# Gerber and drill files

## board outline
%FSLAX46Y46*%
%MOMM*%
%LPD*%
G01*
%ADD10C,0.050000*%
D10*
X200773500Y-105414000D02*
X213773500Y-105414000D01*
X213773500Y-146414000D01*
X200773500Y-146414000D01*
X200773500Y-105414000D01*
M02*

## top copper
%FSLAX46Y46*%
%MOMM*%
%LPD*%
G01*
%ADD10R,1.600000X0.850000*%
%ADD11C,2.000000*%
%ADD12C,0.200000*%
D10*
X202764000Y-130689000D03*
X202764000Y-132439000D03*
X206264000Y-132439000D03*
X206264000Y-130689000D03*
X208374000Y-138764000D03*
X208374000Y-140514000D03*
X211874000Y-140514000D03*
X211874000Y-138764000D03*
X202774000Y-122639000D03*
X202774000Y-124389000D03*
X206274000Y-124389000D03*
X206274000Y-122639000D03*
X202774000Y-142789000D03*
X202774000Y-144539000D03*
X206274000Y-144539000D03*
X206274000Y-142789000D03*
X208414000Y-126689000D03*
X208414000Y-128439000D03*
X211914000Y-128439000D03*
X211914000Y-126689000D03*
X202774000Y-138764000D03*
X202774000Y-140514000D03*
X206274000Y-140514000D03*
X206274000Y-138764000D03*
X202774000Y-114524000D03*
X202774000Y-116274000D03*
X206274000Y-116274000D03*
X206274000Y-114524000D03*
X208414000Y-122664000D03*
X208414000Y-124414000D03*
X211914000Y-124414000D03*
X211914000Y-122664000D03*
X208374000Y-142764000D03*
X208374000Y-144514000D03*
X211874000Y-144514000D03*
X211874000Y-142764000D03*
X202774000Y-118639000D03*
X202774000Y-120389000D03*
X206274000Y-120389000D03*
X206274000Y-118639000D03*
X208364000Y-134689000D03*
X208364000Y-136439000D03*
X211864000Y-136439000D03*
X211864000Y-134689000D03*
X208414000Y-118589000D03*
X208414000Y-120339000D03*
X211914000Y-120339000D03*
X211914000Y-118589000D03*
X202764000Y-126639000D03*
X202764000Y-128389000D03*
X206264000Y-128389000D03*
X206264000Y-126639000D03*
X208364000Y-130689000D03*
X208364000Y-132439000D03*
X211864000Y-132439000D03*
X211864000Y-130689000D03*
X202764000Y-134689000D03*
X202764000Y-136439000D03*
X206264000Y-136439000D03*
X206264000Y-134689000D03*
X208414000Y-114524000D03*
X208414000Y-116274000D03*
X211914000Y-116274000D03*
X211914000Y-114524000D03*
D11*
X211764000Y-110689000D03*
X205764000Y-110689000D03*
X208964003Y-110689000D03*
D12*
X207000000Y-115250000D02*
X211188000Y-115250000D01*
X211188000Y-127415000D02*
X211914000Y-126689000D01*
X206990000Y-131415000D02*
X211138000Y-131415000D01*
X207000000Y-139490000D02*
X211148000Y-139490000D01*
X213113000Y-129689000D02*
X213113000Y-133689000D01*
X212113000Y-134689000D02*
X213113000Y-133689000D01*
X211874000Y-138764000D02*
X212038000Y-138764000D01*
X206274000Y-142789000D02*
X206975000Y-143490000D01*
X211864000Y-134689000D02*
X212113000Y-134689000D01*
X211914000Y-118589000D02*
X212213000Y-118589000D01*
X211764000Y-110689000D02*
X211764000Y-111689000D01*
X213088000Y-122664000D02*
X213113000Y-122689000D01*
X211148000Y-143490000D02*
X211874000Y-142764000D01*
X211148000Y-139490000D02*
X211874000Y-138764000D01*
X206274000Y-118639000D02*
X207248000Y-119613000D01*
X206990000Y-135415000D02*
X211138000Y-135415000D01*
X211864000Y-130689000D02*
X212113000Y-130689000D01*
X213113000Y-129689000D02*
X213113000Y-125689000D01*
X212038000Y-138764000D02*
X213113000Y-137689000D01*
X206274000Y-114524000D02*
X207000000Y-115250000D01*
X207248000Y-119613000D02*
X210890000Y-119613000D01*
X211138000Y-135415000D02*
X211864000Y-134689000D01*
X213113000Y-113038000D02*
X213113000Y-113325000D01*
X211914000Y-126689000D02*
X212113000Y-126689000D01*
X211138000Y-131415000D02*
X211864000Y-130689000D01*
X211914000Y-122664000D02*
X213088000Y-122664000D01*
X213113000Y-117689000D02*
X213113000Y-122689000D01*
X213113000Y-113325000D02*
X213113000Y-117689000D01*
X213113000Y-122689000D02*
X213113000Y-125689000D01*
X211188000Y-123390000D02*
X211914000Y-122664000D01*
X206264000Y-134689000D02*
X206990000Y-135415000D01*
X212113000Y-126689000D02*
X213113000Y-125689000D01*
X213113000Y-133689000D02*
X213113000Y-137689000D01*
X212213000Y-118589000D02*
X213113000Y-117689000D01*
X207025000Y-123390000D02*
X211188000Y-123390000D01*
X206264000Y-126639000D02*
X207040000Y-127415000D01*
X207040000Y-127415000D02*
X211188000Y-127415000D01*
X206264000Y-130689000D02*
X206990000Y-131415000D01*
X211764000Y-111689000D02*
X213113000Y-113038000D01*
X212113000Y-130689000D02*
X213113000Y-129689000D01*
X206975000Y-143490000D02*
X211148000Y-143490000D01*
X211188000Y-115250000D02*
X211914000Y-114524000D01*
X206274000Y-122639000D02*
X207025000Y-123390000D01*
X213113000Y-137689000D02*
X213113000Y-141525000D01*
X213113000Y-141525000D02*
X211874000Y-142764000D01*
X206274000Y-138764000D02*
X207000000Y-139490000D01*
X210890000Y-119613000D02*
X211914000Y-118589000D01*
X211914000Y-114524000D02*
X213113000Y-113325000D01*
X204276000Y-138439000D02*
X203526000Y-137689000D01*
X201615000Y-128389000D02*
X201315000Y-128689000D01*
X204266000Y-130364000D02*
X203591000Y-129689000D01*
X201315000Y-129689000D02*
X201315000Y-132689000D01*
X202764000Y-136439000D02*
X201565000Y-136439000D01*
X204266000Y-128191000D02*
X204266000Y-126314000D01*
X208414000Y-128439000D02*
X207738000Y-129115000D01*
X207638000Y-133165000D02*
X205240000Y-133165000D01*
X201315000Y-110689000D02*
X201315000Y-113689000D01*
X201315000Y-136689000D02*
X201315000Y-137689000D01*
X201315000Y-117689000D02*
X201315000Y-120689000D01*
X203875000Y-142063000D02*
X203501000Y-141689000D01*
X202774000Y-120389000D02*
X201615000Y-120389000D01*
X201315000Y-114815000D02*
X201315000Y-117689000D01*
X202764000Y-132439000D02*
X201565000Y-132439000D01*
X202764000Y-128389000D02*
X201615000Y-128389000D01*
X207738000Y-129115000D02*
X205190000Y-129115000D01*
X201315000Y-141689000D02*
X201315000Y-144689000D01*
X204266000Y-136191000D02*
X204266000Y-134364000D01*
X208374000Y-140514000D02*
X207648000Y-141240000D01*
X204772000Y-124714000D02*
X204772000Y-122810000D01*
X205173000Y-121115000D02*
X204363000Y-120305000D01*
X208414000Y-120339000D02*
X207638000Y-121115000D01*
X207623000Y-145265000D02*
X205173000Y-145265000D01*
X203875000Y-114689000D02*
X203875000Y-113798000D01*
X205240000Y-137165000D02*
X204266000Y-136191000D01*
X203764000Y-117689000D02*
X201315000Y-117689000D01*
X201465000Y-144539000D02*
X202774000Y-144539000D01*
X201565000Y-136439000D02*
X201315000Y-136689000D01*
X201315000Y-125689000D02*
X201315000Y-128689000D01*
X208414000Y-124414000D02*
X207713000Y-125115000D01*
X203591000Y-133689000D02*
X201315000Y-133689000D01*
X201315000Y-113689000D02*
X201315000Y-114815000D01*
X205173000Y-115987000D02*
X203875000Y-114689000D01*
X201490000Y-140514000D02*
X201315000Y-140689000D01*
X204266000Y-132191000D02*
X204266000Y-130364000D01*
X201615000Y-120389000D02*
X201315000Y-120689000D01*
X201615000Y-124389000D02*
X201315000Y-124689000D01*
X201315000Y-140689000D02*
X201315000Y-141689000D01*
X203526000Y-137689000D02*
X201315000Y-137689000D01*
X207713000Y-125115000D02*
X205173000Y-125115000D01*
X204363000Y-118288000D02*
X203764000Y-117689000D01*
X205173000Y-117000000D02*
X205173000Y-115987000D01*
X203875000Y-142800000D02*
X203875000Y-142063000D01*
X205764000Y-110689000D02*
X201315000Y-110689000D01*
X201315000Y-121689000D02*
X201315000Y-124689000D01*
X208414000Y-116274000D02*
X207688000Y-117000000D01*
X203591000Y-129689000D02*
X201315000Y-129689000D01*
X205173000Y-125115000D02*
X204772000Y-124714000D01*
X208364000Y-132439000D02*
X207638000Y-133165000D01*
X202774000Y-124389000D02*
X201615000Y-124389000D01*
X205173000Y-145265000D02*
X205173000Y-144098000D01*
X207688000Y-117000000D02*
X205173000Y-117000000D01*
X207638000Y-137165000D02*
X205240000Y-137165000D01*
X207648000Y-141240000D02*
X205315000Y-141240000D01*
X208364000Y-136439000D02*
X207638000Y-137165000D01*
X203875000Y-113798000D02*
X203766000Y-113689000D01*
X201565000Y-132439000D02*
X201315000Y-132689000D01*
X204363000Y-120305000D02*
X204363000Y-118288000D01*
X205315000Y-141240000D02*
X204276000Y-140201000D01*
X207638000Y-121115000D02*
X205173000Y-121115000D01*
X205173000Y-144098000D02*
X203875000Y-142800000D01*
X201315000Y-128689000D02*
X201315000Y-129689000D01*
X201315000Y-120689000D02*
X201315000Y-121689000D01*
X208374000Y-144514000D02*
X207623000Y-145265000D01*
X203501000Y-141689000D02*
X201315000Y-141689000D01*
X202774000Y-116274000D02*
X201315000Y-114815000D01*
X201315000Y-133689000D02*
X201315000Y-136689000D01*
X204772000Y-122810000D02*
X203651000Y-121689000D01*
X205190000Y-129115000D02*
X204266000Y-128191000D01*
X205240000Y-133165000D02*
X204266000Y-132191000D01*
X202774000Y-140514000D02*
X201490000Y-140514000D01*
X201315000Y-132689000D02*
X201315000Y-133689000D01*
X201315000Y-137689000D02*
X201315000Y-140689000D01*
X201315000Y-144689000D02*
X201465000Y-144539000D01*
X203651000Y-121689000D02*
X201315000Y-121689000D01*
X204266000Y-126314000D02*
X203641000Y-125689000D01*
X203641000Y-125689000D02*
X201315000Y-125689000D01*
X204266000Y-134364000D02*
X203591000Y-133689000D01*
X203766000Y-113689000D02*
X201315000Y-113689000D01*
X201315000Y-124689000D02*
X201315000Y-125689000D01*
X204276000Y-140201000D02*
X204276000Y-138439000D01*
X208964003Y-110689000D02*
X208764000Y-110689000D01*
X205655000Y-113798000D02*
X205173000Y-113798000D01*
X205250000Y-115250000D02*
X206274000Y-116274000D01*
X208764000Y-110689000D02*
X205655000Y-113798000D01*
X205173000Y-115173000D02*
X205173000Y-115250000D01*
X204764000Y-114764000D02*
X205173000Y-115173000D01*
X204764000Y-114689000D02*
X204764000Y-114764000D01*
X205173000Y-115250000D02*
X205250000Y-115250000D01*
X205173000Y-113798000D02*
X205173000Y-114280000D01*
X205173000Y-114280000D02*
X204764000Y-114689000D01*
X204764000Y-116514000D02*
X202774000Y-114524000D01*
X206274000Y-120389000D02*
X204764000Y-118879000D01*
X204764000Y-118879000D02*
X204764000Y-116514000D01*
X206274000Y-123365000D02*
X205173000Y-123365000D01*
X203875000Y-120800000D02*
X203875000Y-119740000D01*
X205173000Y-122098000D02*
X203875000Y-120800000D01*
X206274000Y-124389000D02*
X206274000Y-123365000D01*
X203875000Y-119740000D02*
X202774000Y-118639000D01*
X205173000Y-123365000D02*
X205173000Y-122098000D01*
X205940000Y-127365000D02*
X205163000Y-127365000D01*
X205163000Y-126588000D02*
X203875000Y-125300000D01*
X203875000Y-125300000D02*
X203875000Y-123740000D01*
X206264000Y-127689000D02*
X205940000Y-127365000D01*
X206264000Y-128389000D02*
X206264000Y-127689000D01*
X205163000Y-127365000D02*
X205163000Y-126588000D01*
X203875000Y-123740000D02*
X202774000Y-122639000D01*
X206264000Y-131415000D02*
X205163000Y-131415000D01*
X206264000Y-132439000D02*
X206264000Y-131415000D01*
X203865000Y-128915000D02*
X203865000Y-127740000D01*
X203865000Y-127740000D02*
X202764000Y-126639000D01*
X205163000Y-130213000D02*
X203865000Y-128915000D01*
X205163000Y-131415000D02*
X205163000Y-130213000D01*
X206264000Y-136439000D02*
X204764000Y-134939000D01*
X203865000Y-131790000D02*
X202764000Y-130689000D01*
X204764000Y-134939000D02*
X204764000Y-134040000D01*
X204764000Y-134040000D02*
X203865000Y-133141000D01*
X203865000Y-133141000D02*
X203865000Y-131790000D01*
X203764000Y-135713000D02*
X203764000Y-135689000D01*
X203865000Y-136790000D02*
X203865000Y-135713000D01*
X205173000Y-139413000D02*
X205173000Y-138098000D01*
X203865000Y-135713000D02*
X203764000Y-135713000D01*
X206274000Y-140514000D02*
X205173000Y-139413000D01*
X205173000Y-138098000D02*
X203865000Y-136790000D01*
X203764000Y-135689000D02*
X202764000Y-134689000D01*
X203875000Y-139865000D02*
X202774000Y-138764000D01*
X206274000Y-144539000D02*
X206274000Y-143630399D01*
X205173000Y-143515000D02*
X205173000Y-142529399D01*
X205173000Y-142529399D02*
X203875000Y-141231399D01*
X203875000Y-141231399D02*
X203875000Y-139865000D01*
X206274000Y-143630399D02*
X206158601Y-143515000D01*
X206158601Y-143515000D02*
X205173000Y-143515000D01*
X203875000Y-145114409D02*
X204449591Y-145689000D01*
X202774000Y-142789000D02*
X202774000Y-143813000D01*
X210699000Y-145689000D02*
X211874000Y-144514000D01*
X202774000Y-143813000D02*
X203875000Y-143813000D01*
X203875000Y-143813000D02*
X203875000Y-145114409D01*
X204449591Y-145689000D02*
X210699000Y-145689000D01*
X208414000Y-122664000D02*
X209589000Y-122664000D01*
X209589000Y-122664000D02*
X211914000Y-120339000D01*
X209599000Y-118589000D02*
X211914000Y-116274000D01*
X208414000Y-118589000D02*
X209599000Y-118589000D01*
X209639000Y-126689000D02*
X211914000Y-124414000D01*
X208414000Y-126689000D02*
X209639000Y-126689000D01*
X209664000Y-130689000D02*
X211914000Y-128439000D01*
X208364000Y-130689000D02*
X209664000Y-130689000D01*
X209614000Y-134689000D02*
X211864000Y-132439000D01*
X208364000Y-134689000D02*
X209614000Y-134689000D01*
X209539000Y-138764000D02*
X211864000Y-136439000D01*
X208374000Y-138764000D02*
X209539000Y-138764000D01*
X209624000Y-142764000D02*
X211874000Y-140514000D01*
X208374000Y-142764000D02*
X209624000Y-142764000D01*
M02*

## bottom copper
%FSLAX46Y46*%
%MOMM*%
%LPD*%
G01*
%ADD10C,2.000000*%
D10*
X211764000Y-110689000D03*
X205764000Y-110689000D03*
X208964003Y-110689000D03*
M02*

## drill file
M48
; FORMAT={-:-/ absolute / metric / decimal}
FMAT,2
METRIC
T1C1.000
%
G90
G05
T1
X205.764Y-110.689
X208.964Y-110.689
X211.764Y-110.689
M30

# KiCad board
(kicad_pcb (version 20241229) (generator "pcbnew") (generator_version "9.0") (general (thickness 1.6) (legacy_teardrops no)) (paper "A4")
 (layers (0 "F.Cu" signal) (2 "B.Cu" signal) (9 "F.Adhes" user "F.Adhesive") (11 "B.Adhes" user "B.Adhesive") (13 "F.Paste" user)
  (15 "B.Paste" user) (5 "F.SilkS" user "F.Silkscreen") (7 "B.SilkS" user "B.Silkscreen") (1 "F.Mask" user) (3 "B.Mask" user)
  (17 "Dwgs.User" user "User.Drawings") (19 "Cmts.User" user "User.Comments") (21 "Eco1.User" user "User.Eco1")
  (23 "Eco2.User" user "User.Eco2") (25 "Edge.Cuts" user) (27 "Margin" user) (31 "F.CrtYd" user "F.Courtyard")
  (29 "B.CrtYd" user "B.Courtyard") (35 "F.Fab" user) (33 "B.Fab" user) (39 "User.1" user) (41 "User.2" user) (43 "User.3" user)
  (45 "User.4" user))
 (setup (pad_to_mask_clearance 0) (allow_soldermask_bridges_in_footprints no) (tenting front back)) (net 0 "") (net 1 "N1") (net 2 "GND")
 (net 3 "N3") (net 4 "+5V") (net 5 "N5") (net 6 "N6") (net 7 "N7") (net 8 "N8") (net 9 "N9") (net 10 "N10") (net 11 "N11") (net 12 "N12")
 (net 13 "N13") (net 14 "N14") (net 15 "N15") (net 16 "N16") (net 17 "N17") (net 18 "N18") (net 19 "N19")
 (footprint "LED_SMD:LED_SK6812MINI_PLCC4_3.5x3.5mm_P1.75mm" (layer "F.Cu") (at 204.514 131.564)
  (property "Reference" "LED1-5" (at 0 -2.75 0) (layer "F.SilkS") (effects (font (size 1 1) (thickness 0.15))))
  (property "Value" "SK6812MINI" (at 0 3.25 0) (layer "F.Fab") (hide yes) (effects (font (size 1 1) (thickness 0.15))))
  (pad "1" smd rect (at -1.75 -0.875) (size 1.6 0.85) (layers "F.Cu" "F.Mask" "F.Paste") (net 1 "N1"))
  (pad "2" smd rect (at -1.75 0.875) (size 1.6 0.85) (layers "F.Cu" "F.Mask" "F.Paste") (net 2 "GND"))
  (pad "3" smd rect (at 1.75 0.875) (size 1.6 0.85) (layers "F.Cu" "F.Mask" "F.Paste") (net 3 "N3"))
  (pad "4" smd rect (at 1.75 -0.875) (size 1.6 0.85) (layers "F.Cu" "F.Mask" "F.Paste") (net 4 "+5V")))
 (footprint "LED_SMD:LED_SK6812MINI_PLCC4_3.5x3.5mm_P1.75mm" (layer "F.Cu") (at 210.124 139.639)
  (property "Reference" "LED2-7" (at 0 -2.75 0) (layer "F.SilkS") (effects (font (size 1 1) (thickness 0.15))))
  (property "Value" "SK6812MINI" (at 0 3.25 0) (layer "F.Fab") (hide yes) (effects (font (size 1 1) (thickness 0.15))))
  (pad "1" smd rect (at -1.75 -0.875) (size 1.6 0.85) (layers "F.Cu" "F.Mask" "F.Paste") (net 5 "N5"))
  (pad "2" smd rect (at -1.75 0.875) (size 1.6 0.85) (layers "F.Cu" "F.Mask" "F.Paste") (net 2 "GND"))
  (pad "3" smd rect (at 1.75 0.875) (size 1.6 0.85) (layers "F.Cu" "F.Mask" "F.Paste") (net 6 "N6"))
  (pad "4" smd rect (at 1.75 -0.875) (size 1.6 0.85) (layers "F.Cu" "F.Mask" "F.Paste") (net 4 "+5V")))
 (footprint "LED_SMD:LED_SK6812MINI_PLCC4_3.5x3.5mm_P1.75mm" (layer "F.Cu") (at 204.524 123.514)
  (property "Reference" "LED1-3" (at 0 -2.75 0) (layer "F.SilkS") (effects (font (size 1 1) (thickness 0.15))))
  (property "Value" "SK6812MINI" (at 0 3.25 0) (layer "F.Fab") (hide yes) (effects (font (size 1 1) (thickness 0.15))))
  (pad "1" smd rect (at -1.75 -0.875) (size 1.6 0.85) (layers "F.Cu" "F.Mask" "F.Paste") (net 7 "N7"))
  (pad "2" smd rect (at -1.75 0.875) (size 1.6 0.85) (layers "F.Cu" "F.Mask" "F.Paste") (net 2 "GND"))
  (pad "3" smd rect (at 1.75 0.875) (size 1.6 0.85) (layers "F.Cu" "F.Mask" "F.Paste") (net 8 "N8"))
  (pad "4" smd rect (at 1.75 -0.875) (size 1.6 0.85) (layers "F.Cu" "F.Mask" "F.Paste") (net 4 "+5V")))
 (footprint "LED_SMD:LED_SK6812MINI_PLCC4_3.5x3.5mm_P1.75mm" (layer "F.Cu") (at 204.524 143.664)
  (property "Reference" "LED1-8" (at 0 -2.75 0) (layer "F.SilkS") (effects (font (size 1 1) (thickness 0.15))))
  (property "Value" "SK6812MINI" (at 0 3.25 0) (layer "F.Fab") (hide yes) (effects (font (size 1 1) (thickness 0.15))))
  (pad "1" smd rect (at -1.75 -0.875) (size 1.6 0.85) (layers "F.Cu" "F.Mask" "F.Paste") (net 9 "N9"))
  (pad "2" smd rect (at -1.75 0.875) (size 1.6 0.85) (layers "F.Cu" "F.Mask" "F.Paste") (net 2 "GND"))
  (pad "3" smd rect (at 1.75 0.875) (size 1.6 0.85) (layers "F.Cu" "F.Mask" "F.Paste") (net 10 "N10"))
  (pad "4" smd rect (at 1.75 -0.875) (size 1.6 0.85) (layers "F.Cu" "F.Mask" "F.Paste") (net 4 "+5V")))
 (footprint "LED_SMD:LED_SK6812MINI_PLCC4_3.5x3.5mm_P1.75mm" (layer "F.Cu") (at 210.164 127.564)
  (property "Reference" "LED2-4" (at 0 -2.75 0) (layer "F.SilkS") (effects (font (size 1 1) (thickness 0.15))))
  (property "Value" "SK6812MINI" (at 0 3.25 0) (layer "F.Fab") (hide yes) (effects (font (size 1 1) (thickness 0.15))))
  (pad "1" smd rect (at -1.75 -0.875) (size 1.6 0.85) (layers "F.Cu" "F.Mask" "F.Paste") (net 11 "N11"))
  (pad "2" smd rect (at -1.75 0.875) (size 1.6 0.85) (layers "F.Cu" "F.Mask" "F.Paste") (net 2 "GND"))
  (pad "3" smd rect (at 1.75 0.875) (size 1.6 0.85) (layers "F.Cu" "F.Mask" "F.Paste") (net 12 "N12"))
  (pad "4" smd rect (at 1.75 -0.875) (size 1.6 0.85) (layers "F.Cu" "F.Mask" "F.Paste") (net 4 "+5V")))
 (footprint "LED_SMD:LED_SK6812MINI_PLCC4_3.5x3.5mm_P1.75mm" (layer "F.Cu") (at 204.524 139.639)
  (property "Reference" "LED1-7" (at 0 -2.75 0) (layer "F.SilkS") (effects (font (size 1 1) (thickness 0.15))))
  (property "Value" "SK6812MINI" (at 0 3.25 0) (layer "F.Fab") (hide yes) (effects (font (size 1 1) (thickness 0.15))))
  (pad "1" smd rect (at -1.75 -0.875) (size 1.6 0.85) (layers "F.Cu" "F.Mask" "F.Paste") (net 10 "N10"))
  (pad "2" smd rect (at -1.75 0.875) (size 1.6 0.85) (layers "F.Cu" "F.Mask" "F.Paste") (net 2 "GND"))
  (pad "3" smd rect (at 1.75 0.875) (size 1.6 0.85) (layers "F.Cu" "F.Mask" "F.Paste") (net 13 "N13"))
  (pad "4" smd rect (at 1.75 -0.875) (size 1.6 0.85) (layers "F.Cu" "F.Mask" "F.Paste") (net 4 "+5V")))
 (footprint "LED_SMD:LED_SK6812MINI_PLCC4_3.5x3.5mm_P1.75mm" (layer "F.Cu") (at 204.524 115.399)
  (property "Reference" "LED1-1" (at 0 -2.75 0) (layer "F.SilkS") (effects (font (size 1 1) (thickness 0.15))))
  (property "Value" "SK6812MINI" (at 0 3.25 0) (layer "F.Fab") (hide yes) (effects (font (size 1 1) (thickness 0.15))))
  (pad "1" smd rect (at -1.75 -0.875) (size 1.6 0.85) (layers "F.Cu" "F.Mask" "F.Paste") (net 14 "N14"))
  (pad "2" smd rect (at -1.75 0.875) (size 1.6 0.85) (layers "F.Cu" "F.Mask" "F.Paste") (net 2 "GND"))
  (pad "3" smd rect (at 1.75 0.875) (size 1.6 0.85) (layers "F.Cu" "F.Mask" "F.Paste") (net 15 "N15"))
  (pad "4" smd rect (at 1.75 -0.875) (size 1.6 0.85) (layers "F.Cu" "F.Mask" "F.Paste") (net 4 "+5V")))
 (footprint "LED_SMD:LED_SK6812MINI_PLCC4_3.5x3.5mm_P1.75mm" (layer "F.Cu") (at 210.164 123.539)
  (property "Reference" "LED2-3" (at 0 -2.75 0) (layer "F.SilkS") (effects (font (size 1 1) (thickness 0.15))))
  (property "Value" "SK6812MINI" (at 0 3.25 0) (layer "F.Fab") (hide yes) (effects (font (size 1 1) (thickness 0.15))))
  (pad "1" smd rect (at -1.75 -0.875) (size 1.6 0.85) (layers "F.Cu" "F.Mask" "F.Paste") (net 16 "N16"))
  (pad "2" smd rect (at -1.75 0.875) (size 1.6 0.85) (layers "F.Cu" "F.Mask" "F.Paste") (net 2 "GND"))
  (pad "3" smd rect (at 1.75 0.875) (size 1.6 0.85) (layers "F.Cu" "F.Mask" "F.Paste") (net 11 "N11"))
  (pad "4" smd rect (at 1.75 -0.875) (size 1.6 0.85) (layers "F.Cu" "F.Mask" "F.Paste") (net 4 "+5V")))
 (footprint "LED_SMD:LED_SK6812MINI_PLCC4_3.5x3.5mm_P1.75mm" (layer "F.Cu") (at 210.124 143.639)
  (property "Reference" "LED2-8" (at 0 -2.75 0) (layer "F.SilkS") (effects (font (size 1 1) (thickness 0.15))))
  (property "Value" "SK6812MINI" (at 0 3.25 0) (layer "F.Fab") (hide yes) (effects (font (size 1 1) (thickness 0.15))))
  (pad "1" smd rect (at -1.75 -0.875) (size 1.6 0.85) (layers "F.Cu" "F.Mask" "F.Paste") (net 6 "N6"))
  (pad "2" smd rect (at -1.75 0.875) (size 1.6 0.85) (layers "F.Cu" "F.Mask" "F.Paste") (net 2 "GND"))
  (pad "3" smd rect (at 1.75 0.875) (size 1.6 0.85) (layers "F.Cu" "F.Mask" "F.Paste") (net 9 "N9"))
  (pad "4" smd rect (at 1.75 -0.875) (size 1.6 0.85) (layers "F.Cu" "F.Mask" "F.Paste") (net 4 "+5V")))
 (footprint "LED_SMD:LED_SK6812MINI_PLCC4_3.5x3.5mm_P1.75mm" (layer "F.Cu") (at 204.524 119.514)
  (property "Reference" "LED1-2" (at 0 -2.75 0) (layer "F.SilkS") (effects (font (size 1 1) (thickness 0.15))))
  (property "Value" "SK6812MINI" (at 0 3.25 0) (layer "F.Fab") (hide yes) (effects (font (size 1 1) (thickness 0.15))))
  (pad "1" smd rect (at -1.75 -0.875) (size 1.6 0.85) (layers "F.Cu" "F.Mask" "F.Paste") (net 8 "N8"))
  (pad "2" smd rect (at -1.75 0.875) (size 1.6 0.85) (layers "F.Cu" "F.Mask" "F.Paste") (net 2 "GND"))
  (pad "3" smd rect (at 1.75 0.875) (size 1.6 0.85) (layers "F.Cu" "F.Mask" "F.Paste") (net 14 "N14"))
  (pad "4" smd rect (at 1.75 -0.875) (size 1.6 0.85) (layers "F.Cu" "F.Mask" "F.Paste") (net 4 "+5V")))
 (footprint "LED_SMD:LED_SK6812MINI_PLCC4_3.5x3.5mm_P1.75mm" (layer "F.Cu") (at 210.114 135.564)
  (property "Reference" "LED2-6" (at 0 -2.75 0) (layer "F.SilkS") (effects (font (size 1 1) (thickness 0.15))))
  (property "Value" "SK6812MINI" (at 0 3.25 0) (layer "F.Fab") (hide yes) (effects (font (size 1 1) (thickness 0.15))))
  (pad "1" smd rect (at -1.75 -0.875) (size 1.6 0.85) (layers "F.Cu" "F.Mask" "F.Paste") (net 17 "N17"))
  (pad "2" smd rect (at -1.75 0.875) (size 1.6 0.85) (layers "F.Cu" "F.Mask" "F.Paste") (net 2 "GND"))
  (pad "3" smd rect (at 1.75 0.875) (size 1.6 0.85) (layers "F.Cu" "F.Mask" "F.Paste") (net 5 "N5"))
  (pad "4" smd rect (at 1.75 -0.875) (size 1.6 0.85) (layers "F.Cu" "F.Mask" "F.Paste") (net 4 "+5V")))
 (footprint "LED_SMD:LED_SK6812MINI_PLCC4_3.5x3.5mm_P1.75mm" (layer "F.Cu") (at 210.164 119.464)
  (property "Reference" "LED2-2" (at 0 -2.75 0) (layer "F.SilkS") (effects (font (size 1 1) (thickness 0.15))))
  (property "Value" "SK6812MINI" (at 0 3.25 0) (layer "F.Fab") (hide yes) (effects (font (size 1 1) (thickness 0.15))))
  (pad "1" smd rect (at -1.75 -0.875) (size 1.6 0.85) (layers "F.Cu" "F.Mask" "F.Paste") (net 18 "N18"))
  (pad "2" smd rect (at -1.75 0.875) (size 1.6 0.85) (layers "F.Cu" "F.Mask" "F.Paste") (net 2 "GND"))
  (pad "3" smd rect (at 1.75 0.875) (size 1.6 0.85) (layers "F.Cu" "F.Mask" "F.Paste") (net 16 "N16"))
  (pad "4" smd rect (at 1.75 -0.875) (size 1.6 0.85) (layers "F.Cu" "F.Mask" "F.Paste") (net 4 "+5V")))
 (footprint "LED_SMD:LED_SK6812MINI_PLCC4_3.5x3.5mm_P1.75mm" (layer "F.Cu") (at 204.514 127.514)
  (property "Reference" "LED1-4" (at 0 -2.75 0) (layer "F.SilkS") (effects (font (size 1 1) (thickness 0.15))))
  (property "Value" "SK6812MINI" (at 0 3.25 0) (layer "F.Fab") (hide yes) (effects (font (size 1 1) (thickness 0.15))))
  (pad "1" smd rect (at -1.75 -0.875) (size 1.6 0.85) (layers "F.Cu" "F.Mask" "F.Paste") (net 3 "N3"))
  (pad "2" smd rect (at -1.75 0.875) (size 1.6 0.85) (layers "F.Cu" "F.Mask" "F.Paste") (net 2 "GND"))
  (pad "3" smd rect (at 1.75 0.875) (size 1.6 0.85) (layers "F.Cu" "F.Mask" "F.Paste") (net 7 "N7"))
  (pad "4" smd rect (at 1.75 -0.875) (size 1.6 0.85) (layers "F.Cu" "F.Mask" "F.Paste") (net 4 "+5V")))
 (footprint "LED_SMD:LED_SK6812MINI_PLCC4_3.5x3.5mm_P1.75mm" (layer "F.Cu") (at 210.114 131.564)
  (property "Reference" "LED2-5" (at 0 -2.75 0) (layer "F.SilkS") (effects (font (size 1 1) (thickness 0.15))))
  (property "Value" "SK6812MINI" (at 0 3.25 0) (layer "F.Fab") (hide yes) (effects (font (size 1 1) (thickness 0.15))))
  (pad "1" smd rect (at -1.75 -0.875) (size 1.6 0.85) (layers "F.Cu" "F.Mask" "F.Paste") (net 12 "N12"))
  (pad "2" smd rect (at -1.75 0.875) (size 1.6 0.85) (layers "F.Cu" "F.Mask" "F.Paste") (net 2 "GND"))
  (pad "3" smd rect (at 1.75 0.875) (size 1.6 0.85) (layers "F.Cu" "F.Mask" "F.Paste") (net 17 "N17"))
  (pad "4" smd rect (at 1.75 -0.875) (size 1.6 0.85) (layers "F.Cu" "F.Mask" "F.Paste") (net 4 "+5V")))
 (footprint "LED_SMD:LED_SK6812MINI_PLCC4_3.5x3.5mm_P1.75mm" (layer "F.Cu") (at 204.514 135.564)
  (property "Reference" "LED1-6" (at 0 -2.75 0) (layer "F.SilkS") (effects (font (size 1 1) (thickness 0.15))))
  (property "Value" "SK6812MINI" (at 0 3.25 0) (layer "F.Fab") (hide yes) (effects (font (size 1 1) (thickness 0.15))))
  (pad "1" smd rect (at -1.75 -0.875) (size 1.6 0.85) (layers "F.Cu" "F.Mask" "F.Paste") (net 13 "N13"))
  (pad "2" smd rect (at -1.75 0.875) (size 1.6 0.85) (layers "F.Cu" "F.Mask" "F.Paste") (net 2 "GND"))
  (pad "3" smd rect (at 1.75 0.875) (size 1.6 0.85) (layers "F.Cu" "F.Mask" "F.Paste") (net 1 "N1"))
  (pad "4" smd rect (at 1.75 -0.875) (size 1.6 0.85) (layers "F.Cu" "F.Mask" "F.Paste") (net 4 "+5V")))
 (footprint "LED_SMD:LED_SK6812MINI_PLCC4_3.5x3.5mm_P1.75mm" (layer "F.Cu") (at 210.164 115.399)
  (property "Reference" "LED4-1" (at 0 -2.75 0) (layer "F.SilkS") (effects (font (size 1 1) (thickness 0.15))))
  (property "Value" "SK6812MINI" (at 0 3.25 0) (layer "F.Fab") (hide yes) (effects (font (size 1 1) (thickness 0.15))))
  (pad "1" smd rect (at -1.75 -0.875) (size 1.6 0.85) (layers "F.Cu" "F.Mask" "F.Paste") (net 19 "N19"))
  (pad "2" smd rect (at -1.75 0.875) (size 1.6 0.85) (layers "F.Cu" "F.Mask" "F.Paste") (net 2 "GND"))
  (pad "3" smd rect (at 1.75 0.875) (size 1.6 0.85) (layers "F.Cu" "F.Mask" "F.Paste") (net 18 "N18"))
  (pad "4" smd rect (at 1.75 -0.875) (size 1.6 0.85) (layers "F.Cu" "F.Mask" "F.Paste") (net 4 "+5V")))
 (gr_rect (start 200.7735 105.414) (end 213.7735 146.414) (stroke (width 0.05) (type default)) (fill no) (layer "Edge.Cuts"))
 (segment (start 207 115.25) (end 211.188 115.25) (width 0.2) (layer "F.Cu") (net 4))
 (segment (start 211.188 127.415) (end 211.914 126.689) (width 0.2) (layer "F.Cu") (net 4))
 (segment (start 206.99 131.415) (end 211.138 131.415) (width 0.2) (layer "F.Cu") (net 4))
 (segment (start 207 139.49) (end 211.148 139.49) (width 0.2) (layer "F.Cu") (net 4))
 (segment (start 213.113 129.689) (end 213.113 133.689) (width 0.2) (layer "F.Cu") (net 4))
 (segment (start 212.113 134.689) (end 213.113 133.689) (width 0.2) (layer "F.Cu") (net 4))
 (segment (start 211.874 138.764) (end 212.038 138.764) (width 0.2) (layer "F.Cu") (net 4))
 (segment (start 206.274 142.789) (end 206.975 143.49) (width 0.2) (layer "F.Cu") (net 4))
 (segment (start 211.864 134.689) (end 212.113 134.689) (width 0.2) (layer "F.Cu") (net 4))
 (segment (start 211.914 118.589) (end 212.213 118.589) (width 0.2) (layer "F.Cu") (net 4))
 (segment (start 211.764 110.689) (end 211.764 111.689) (width 0.2) (layer "F.Cu") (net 4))
 (segment (start 213.088 122.664) (end 213.113 122.689) (width 0.2) (layer "F.Cu") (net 4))
 (segment (start 211.148 143.49) (end 211.874 142.764) (width 0.2) (layer "F.Cu") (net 4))
 (segment (start 211.148 139.49) (end 211.874 138.764) (width 0.2) (layer "F.Cu") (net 4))
 (segment (start 206.274 118.639) (end 207.248 119.613) (width 0.2) (layer "F.Cu") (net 4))
 (segment (start 206.99 135.415) (end 211.138 135.415) (width 0.2) (layer "F.Cu") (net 4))
 (segment (start 211.864 130.689) (end 212.113 130.689) (width 0.2) (layer "F.Cu") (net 4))
 (segment (start 213.113 129.689) (end 213.113 125.689) (width 0.2) (layer "F.Cu") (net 4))
 (segment (start 212.038 138.764) (end 213.113 137.689) (width 0.2) (layer "F.Cu") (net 4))
 (segment (start 206.274 114.524) (end 207 115.25) (width 0.2) (layer "F.Cu") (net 4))
 (segment (start 207.248 119.613) (end 210.89 119.613) (width 0.2) (layer "F.Cu") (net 4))
 (segment (start 211.138 135.415) (end 211.864 134.689) (width 0.2) (layer "F.Cu") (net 4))
 (segment (start 213.113 113.038) (end 213.113 113.325) (width 0.2) (layer "F.Cu") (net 4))
 (segment (start 211.914 126.689) (end 212.113 126.689) (width 0.2) (layer "F.Cu") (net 4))
 (segment (start 211.138 131.415) (end 211.864 130.689) (width 0.2) (layer "F.Cu") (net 4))
 (segment (start 211.914 122.664) (end 213.088 122.664) (width 0.2) (layer "F.Cu") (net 4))
 (segment (start 213.113 117.689) (end 213.113 122.689) (width 0.2) (layer "F.Cu") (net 4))
 (segment (start 213.113 113.325) (end 213.113 117.689) (width 0.2) (layer "F.Cu") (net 4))
 (segment (start 213.113 122.689) (end 213.113 125.689) (width 0.2) (layer "F.Cu") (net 4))
 (segment (start 211.188 123.39) (end 211.914 122.664) (width 0.2) (layer "F.Cu") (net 4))
 (segment (start 206.264 134.689) (end 206.99 135.415) (width 0.2) (layer "F.Cu") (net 4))
 (segment (start 212.113 126.689) (end 213.113 125.689) (width 0.2) (layer "F.Cu") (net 4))
 (segment (start 213.113 133.689) (end 213.113 137.689) (width 0.2) (layer "F.Cu") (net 4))
 (segment (start 212.213 118.589) (end 213.113 117.689) (width 0.2) (layer "F.Cu") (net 4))
 (segment (start 207.025 123.39) (end 211.188 123.39) (width 0.2) (layer "F.Cu") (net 4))
 (segment (start 206.264 126.639) (end 207.04 127.415) (width 0.2) (layer "F.Cu") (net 4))
 (segment (start 207.04 127.415) (end 211.188 127.415) (width 0.2) (layer "F.Cu") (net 4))
 (segment (start 206.264 130.689) (end 206.99 131.415) (width 0.2) (layer "F.Cu") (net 4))
 (segment (start 211.764 111.689) (end 213.113 113.038) (width 0.2) (layer "F.Cu") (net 4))
 (segment (start 212.113 130.689) (end 213.113 129.689) (width 0.2) (layer "F.Cu") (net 4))
 (segment (start 206.975 143.49) (end 211.148 143.49) (width 0.2) (layer "F.Cu") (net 4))
 (segment (start 211.188 115.25) (end 211.914 114.524) (width 0.2) (layer "F.Cu") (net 4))
 (segment (start 206.274 122.639) (end 207.025 123.39) (width 0.2) (layer "F.Cu") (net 4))
 (segment (start 213.113 137.689) (end 213.113 141.525) (width 0.2) (layer "F.Cu") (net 4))
 (segment (start 213.113 141.525) (end 211.874 142.764) (width 0.2) (layer "F.Cu") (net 4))
 (segment (start 206.274 138.764) (end 207 139.49) (width 0.2) (layer "F.Cu") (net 4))
 (segment (start 210.89 119.613) (end 211.914 118.589) (width 0.2) (layer "F.Cu") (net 4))
 (segment (start 211.914 114.524) (end 213.113 113.325) (width 0.2) (layer "F.Cu") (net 4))
 (via (at 211.764 110.689) (size 2) (drill 1) (layers "F.Cu" "B.Cu") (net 4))
 (segment (start 204.276 138.439) (end 203.526 137.689) (width 0.2) (layer "F.Cu") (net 2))
 (segment (start 201.615 128.389) (end 201.315 128.689) (width 0.2) (layer "F.Cu") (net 2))
 (segment (start 204.266 130.364) (end 203.591 129.689) (width 0.2) (layer "F.Cu") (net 2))
 (segment (start 201.315 129.689) (end 201.315 132.689) (width 0.2) (layer "F.Cu") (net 2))
 (segment (start 202.764 136.439) (end 201.565 136.439) (width 0.2) (layer "F.Cu") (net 2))
 (segment (start 204.266 128.191) (end 204.266 126.314) (width 0.2) (layer "F.Cu") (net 2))
 (segment (start 208.414 128.439) (end 207.738 129.115) (width 0.2) (layer "F.Cu") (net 2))
 (segment (start 207.638 133.165) (end 205.24 133.165) (width 0.2) (layer "F.Cu") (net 2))
 (segment (start 201.315 110.689) (end 201.315 113.689) (width 0.2) (layer "F.Cu") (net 2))
 (segment (start 201.315 136.689) (end 201.315 137.689) (width 0.2) (layer "F.Cu") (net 2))
 (segment (start 201.315 117.689) (end 201.315 120.689) (width 0.2) (layer "F.Cu") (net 2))
 (segment (start 203.875 142.063) (end 203.501 141.689) (width 0.2) (layer "F.Cu") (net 2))
 (segment (start 202.774 120.389) (end 201.615 120.389) (width 0.2) (layer "F.Cu") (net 2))
 (segment (start 201.315 114.815) (end 201.315 117.689) (width 0.2) (layer "F.Cu") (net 2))
 (segment (start 202.764 132.439) (end 201.565 132.439) (width 0.2) (layer "F.Cu") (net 2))
 (segment (start 202.764 128.389) (end 201.615 128.389) (width 0.2) (layer "F.Cu") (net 2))
 (segment (start 207.738 129.115) (end 205.19 129.115) (width 0.2) (layer "F.Cu") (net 2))
 (segment (start 201.315 141.689) (end 201.315 144.689) (width 0.2) (layer "F.Cu") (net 2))
 (segment (start 204.266 136.191) (end 204.266 134.364) (width 0.2) (layer "F.Cu") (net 2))
 (segment (start 208.374 140.514) (end 207.648 141.24) (width 0.2) (layer "F.Cu") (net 2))
 (segment (start 204.772 124.714) (end 204.772 122.81) (width 0.2) (layer "F.Cu") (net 2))
 (segment (start 205.173 121.115) (end 204.363 120.305) (width 0.2) (layer "F.Cu") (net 2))
 (segment (start 208.414 120.339) (end 207.638 121.115) (width 0.2) (layer "F.Cu") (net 2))
 (segment (start 207.623 145.265) (end 205.173 145.265) (width 0.2) (layer "F.Cu") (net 2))
 (segment (start 203.875 114.689) (end 203.875 113.798) (width 0.2) (layer "F.Cu") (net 2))
 (segment (start 205.24 137.165) (end 204.266 136.191) (width 0.2) (layer "F.Cu") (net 2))
 (segment (start 203.764 117.689) (end 201.315 117.689) (width 0.2) (layer "F.Cu") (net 2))
 (segment (start 201.465 144.539) (end 202.774 144.539) (width 0.2) (layer "F.Cu") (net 2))
 (segment (start 201.565 136.439) (end 201.315 136.689) (width 0.2) (layer "F.Cu") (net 2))
 (segment (start 201.315 125.689) (end 201.315 128.689) (width 0.2) (layer "F.Cu") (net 2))
 (segment (start 208.414 124.414) (end 207.713 125.115) (width 0.2) (layer "F.Cu") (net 2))
 (segment (start 203.591 133.689) (end 201.315 133.689) (width 0.2) (layer "F.Cu") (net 2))
 (segment (start 201.315 113.689) (end 201.315 114.815) (width 0.2) (layer "F.Cu") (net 2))
 (segment (start 205.173 115.987) (end 203.875 114.689) (width 0.2) (layer "F.Cu") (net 2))
 (segment (start 201.49 140.514) (end 201.315 140.689) (width 0.2) (layer "F.Cu") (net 2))
 (segment (start 204.266 132.191) (end 204.266 130.364) (width 0.2) (layer "F.Cu") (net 2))
 (segment (start 201.615 120.389) (end 201.315 120.689) (width 0.2) (layer "F.Cu") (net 2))
 (segment (start 201.615 124.389) (end 201.315 124.689) (width 0.2) (layer "F.Cu") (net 2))
 (segment (start 201.315 140.689) (end 201.315 141.689) (width 0.2) (layer "F.Cu") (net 2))
 (segment (start 203.526 137.689) (end 201.315 137.689) (width 0.2) (layer "F.Cu") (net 2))
 (segment (start 207.713 125.115) (end 205.173 125.115) (width 0.2) (layer "F.Cu") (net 2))
 (segment (start 204.363 118.288) (end 203.764 117.689) (width 0.2) (layer "F.Cu") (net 2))
 (segment (start 205.173 117) (end 205.173 115.987) (width 0.2) (layer "F.Cu") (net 2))
 (segment (start 203.875 142.8) (end 203.875 142.063) (width 0.2) (layer "F.Cu") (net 2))
 (segment (start 205.764 110.689) (end 201.315 110.689) (width 0.2) (layer "F.Cu") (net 2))
 (segment (start 201.315 121.689) (end 201.315 124.689) (width 0.2) (layer "F.Cu") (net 2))
 (segment (start 208.414 116.274) (end 207.688 117) (width 0.2) (layer "F.Cu") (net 2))
 (segment (start 203.591 129.689) (end 201.315 129.689) (width 0.2) (layer "F.Cu") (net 2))
 (segment (start 205.173 125.115) (end 204.772 124.714) (width 0.2) (layer "F.Cu") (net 2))
 (segment (start 208.364 132.439) (end 207.638 133.165) (width 0.2) (layer "F.Cu") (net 2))
 (segment (start 202.774 124.389) (end 201.615 124.389) (width 0.2) (layer "F.Cu") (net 2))
 (segment (start 205.173 145.265) (end 205.173 144.098) (width 0.2) (layer "F.Cu") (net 2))
 (segment (start 207.688 117) (end 205.173 117) (width 0.2) (layer "F.Cu") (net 2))
 (segment (start 207.638 137.165) (end 205.24 137.165) (width 0.2) (layer "F.Cu") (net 2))
 (segment (start 207.648 141.24) (end 205.315 141.24) (width 0.2) (layer "F.Cu") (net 2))
 (segment (start 208.364 136.439) (end 207.638 137.165) (width 0.2) (layer "F.Cu") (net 2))
 (segment (start 203.875 113.798) (end 203.766 113.689) (width 0.2) (layer "F.Cu") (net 2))
 (segment (start 201.565 132.439) (end 201.315 132.689) (width 0.2) (layer "F.Cu") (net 2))
 (segment (start 204.363 120.305) (end 204.363 118.288) (width 0.2) (layer "F.Cu") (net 2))
 (segment (start 205.315 141.24) (end 204.276 140.201) (width 0.2) (layer "F.Cu") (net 2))
 (segment (start 207.638 121.115) (end 205.173 121.115) (width 0.2) (layer "F.Cu") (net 2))
 (segment (start 205.173 144.098) (end 203.875 142.8) (width 0.2) (layer "F.Cu") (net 2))
 (segment (start 201.315 128.689) (end 201.315 129.689) (width 0.2) (layer "F.Cu") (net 2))
 (segment (start 201.315 120.689) (end 201.315 121.689) (width 0.2) (layer "F.Cu") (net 2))
 (segment (start 208.374 144.514) (end 207.623 145.265) (width 0.2) (layer "F.Cu") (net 2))
 (segment (start 203.501 141.689) (end 201.315 141.689) (width 0.2) (layer "F.Cu") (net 2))
 (segment (start 202.774 116.274) (end 201.315 114.815) (width 0.2) (layer "F.Cu") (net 2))
 (segment (start 201.315 133.689) (end 201.315 136.689) (width 0.2) (layer "F.Cu") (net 2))
 (segment (start 204.772 122.81) (end 203.651 121.689) (width 0.2) (layer "F.Cu") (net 2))
 (segment (start 205.19 129.115) (end 204.266 128.191) (width 0.2) (layer "F.Cu") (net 2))
 (segment (start 205.24 133.165) (end 204.266 132.191) (width 0.2) (layer "F.Cu") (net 2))
 (segment (start 202.774 140.514) (end 201.49 140.514) (width 0.2) (layer "F.Cu") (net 2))
 (segment (start 201.315 132.689) (end 201.315 133.689) (width 0.2) (layer "F.Cu") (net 2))
 (segment (start 201.315 137.689) (end 201.315 140.689) (width 0.2) (layer "F.Cu") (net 2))
 (segment (start 201.315 144.689) (end 201.465 144.539) (width 0.2) (layer "F.Cu") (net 2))
 (segment (start 203.651 121.689) (end 201.315 121.689) (width 0.2) (layer "F.Cu") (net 2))
 (segment (start 204.266 126.314) (end 203.641 125.689) (width 0.2) (layer "F.Cu") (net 2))
 (segment (start 203.641 125.689) (end 201.315 125.689) (width 0.2) (layer "F.Cu") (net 2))
 (segment (start 204.266 134.364) (end 203.591 133.689) (width 0.2) (layer "F.Cu") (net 2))
 (segment (start 203.766 113.689) (end 201.315 113.689) (width 0.2) (layer "F.Cu") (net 2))
 (segment (start 201.315 124.689) (end 201.315 125.689) (width 0.2) (layer "F.Cu") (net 2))
 (segment (start 204.276 140.201) (end 204.276 138.439) (width 0.2) (layer "F.Cu") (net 2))
 (via (at 205.764 110.689) (size 2) (drill 1) (layers "F.Cu" "B.Cu") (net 2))
 (segment (start 208.964003 110.689) (end 208.764 110.689) (width 0.2) (layer "F.Cu") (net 15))
 (segment (start 205.655 113.798) (end 205.173 113.798) (width 0.2) (layer "F.Cu") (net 15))
 (segment (start 205.25 115.25) (end 206.274 116.274) (width 0.2) (layer "F.Cu") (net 15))
 (segment (start 208.764 110.689) (end 205.655 113.798) (width 0.2) (layer "F.Cu") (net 15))
 (segment (start 205.173 115.173) (end 205.173 115.25) (width 0.2) (layer "F.Cu") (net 15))
 (segment (start 204.764 114.764) (end 205.173 115.173) (width 0.2) (layer "F.Cu") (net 15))
 (segment (start 204.764 114.689) (end 204.764 114.764) (width 0.2) (layer "F.Cu") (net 15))
 (segment (start 205.173 115.25) (end 205.25 115.25) (width 0.2) (layer "F.Cu") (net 15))
 (segment (start 205.173 113.798) (end 205.173 114.28) (width 0.2) (layer "F.Cu") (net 15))
 (segment (start 205.173 114.28) (end 204.764 114.689) (width 0.2) (layer "F.Cu") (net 15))
 (via (at 208.964003 110.689) (size 2) (drill 1) (layers "F.Cu" "B.Cu") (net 15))
 (segment (start 204.764 116.514) (end 202.774 114.524) (width 0.2) (layer "F.Cu") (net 14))
 (segment (start 206.274 120.389) (end 204.764 118.879) (width 0.2) (layer "F.Cu") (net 14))
 (segment (start 204.764 118.879) (end 204.764 116.514) (width 0.2) (layer "F.Cu") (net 14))
 (segment (start 206.274 123.365) (end 205.173 123.365) (width 0.2) (layer "F.Cu") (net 8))
 (segment (start 203.875 120.8) (end 203.875 119.74) (width 0.2) (layer "F.Cu") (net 8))
 (segment (start 205.173 122.098) (end 203.875 120.8) (width 0.2) (layer "F.Cu") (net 8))
 (segment (start 206.274 124.389) (end 206.274 123.365) (width 0.2) (layer "F.Cu") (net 8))
 (segment (start 203.875 119.74) (end 202.774 118.639) (width 0.2) (layer "F.Cu") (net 8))
 (segment (start 205.173 123.365) (end 205.173 122.098) (width 0.2) (layer "F.Cu") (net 8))
 (segment (start 205.94 127.365) (end 205.163 127.365) (width 0.2) (layer "F.Cu") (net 7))
 (segment (start 205.163 126.588) (end 203.875 125.3) (width 0.2) (layer "F.Cu") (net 7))
 (segment (start 203.875 125.3) (end 203.875 123.74) (width 0.2) (layer "F.Cu") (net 7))
 (segment (start 206.264 127.689) (end 205.94 127.365) (width 0.2) (layer "F.Cu") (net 7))
 (segment (start 206.264 128.389) (end 206.264 127.689) (width 0.2) (layer "F.Cu") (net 7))
 (segment (start 205.163 127.365) (end 205.163 126.588) (width 0.2) (layer "F.Cu") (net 7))
 (segment (start 203.875 123.74) (end 202.774 122.639) (width 0.2) (layer "F.Cu") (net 7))
 (segment (start 206.264 131.415) (end 205.163 131.415) (width 0.2) (layer "F.Cu") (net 3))
 (segment (start 206.264 132.439) (end 206.264 131.415) (width 0.2) (layer "F.Cu") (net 3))
 (segment (start 203.865 128.915) (end 203.865 127.74) (width 0.2) (layer "F.Cu") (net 3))
 (segment (start 203.865 127.74) (end 202.764 126.639) (width 0.2) (layer "F.Cu") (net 3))
 (segment (start 205.163 130.213) (end 203.865 128.915) (width 0.2) (layer "F.Cu") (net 3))
 (segment (start 205.163 131.415) (end 205.163 130.213) (width 0.2) (layer "F.Cu") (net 3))
 (segment (start 206.264 136.439) (end 204.764 134.939) (width 0.2) (layer "F.Cu") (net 1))
 (segment (start 203.865 131.79) (end 202.764 130.689) (width 0.2) (layer "F.Cu") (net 1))
 (segment (start 204.764 134.939) (end 204.764 134.04) (width 0.2) (layer "F.Cu") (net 1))
 (segment (start 204.764 134.04) (end 203.865 133.141) (width 0.2) (layer "F.Cu") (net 1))
 (segment (start 203.865 133.141) (end 203.865 131.79) (width 0.2) (layer "F.Cu") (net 1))
 (segment (start 203.764 135.713) (end 203.764 135.689) (width 0.2) (layer "F.Cu") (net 13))
 (segment (start 203.865 136.79) (end 203.865 135.713) (width 0.2) (layer "F.Cu") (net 13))
 (segment (start 205.173 139.413) (end 205.173 138.098) (width 0.2) (layer "F.Cu") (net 13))
 (segment (start 203.865 135.713) (end 203.764 135.713) (width 0.2) (layer "F.Cu") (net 13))
 (segment (start 206.274 140.514) (end 205.173 139.413) (width 0.2) (layer "F.Cu") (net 13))
 (segment (start 205.173 138.098) (end 203.865 136.79) (width 0.2) (layer "F.Cu") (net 13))
 (segment (start 203.764 135.689) (end 202.764 134.689) (width 0.2) (layer "F.Cu") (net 13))
 (segment (start 203.875 139.865) (end 202.774 138.764) (width 0.2) (layer "F.Cu") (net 10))
 (segment (start 206.274 144.539) (end 206.274 143.630399) (width 0.2) (layer "F.Cu") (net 10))
 (segment (start 205.173 143.515) (end 205.173 142.529399) (width 0.2) (layer "F.Cu") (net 10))
 (segment (start 205.173 142.529399) (end 203.875 141.231399) (width 0.2) (layer "F.Cu") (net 10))
 (segment (start 203.875 141.231399) (end 203.875 139.865) (width 0.2) (layer "F.Cu") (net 10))
 (segment (start 206.274 143.630399) (end 206.158601 143.515) (width 0.2) (layer "F.Cu") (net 10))
 (segment (start 206.158601 143.515) (end 205.173 143.515) (width 0.2) (layer "F.Cu") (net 10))
 (segment (start 203.875 145.114409) (end 204.449591 145.689) (width 0.2) (layer "F.Cu") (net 9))
 (segment (start 202.774 142.789) (end 202.774 143.813) (width 0.2) (layer "F.Cu") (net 9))
 (segment (start 210.699 145.689) (end 211.874 144.514) (width 0.2) (layer "F.Cu") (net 9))
 (segment (start 202.774 143.813) (end 203.875 143.813) (width 0.2) (layer "F.Cu") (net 9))
 (segment (start 203.875 143.813) (end 203.875 145.114409) (width 0.2) (layer "F.Cu") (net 9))
 (segment (start 204.449591 145.689) (end 210.699 145.689) (width 0.2) (layer "F.Cu") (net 9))
 (segment (start 208.414 122.664) (end 209.589 122.664) (width 0.2) (layer "F.Cu") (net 16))
 (segment (start 209.589 122.664) (end 211.914 120.339) (width 0.2) (layer "F.Cu") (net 16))
 (segment (start 209.599 118.589) (end 211.914 116.274) (width 0.2) (layer "F.Cu") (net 18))
 (segment (start 208.414 118.589) (end 209.599 118.589) (width 0.2) (layer "F.Cu") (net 18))
 (segment (start 209.639 126.689) (end 211.914 124.414) (width 0.2) (layer "F.Cu") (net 11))
 (segment (start 208.414 126.689) (end 209.639 126.689) (width 0.2) (layer "F.Cu") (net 11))
 (segment (start 209.664 130.689) (end 211.914 128.439) (width 0.2) (layer "F.Cu") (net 12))
 (segment (start 208.364 130.689) (end 209.664 130.689) (width 0.2) (layer "F.Cu") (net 12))
 (segment (start 209.614 134.689) (end 211.864 132.439) (width 0.2) (layer "F.Cu") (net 17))
 (segment (start 208.364 134.689) (end 209.614 134.689) (width 0.2) (layer "F.Cu") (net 17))
 (segment (start 209.539 138.764) (end 211.864 136.439) (width 0.2) (layer "F.Cu") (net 5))
 (segment (start 208.374 138.764) (end 209.539 138.764) (width 0.2) (layer "F.Cu") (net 5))
 (segment (start 209.624 142.764) (end 211.874 140.514) (width 0.2) (layer "F.Cu") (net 6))
 (segment (start 208.374 142.764) (end 209.624 142.764) (width 0.2) (layer "F.Cu") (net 6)))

